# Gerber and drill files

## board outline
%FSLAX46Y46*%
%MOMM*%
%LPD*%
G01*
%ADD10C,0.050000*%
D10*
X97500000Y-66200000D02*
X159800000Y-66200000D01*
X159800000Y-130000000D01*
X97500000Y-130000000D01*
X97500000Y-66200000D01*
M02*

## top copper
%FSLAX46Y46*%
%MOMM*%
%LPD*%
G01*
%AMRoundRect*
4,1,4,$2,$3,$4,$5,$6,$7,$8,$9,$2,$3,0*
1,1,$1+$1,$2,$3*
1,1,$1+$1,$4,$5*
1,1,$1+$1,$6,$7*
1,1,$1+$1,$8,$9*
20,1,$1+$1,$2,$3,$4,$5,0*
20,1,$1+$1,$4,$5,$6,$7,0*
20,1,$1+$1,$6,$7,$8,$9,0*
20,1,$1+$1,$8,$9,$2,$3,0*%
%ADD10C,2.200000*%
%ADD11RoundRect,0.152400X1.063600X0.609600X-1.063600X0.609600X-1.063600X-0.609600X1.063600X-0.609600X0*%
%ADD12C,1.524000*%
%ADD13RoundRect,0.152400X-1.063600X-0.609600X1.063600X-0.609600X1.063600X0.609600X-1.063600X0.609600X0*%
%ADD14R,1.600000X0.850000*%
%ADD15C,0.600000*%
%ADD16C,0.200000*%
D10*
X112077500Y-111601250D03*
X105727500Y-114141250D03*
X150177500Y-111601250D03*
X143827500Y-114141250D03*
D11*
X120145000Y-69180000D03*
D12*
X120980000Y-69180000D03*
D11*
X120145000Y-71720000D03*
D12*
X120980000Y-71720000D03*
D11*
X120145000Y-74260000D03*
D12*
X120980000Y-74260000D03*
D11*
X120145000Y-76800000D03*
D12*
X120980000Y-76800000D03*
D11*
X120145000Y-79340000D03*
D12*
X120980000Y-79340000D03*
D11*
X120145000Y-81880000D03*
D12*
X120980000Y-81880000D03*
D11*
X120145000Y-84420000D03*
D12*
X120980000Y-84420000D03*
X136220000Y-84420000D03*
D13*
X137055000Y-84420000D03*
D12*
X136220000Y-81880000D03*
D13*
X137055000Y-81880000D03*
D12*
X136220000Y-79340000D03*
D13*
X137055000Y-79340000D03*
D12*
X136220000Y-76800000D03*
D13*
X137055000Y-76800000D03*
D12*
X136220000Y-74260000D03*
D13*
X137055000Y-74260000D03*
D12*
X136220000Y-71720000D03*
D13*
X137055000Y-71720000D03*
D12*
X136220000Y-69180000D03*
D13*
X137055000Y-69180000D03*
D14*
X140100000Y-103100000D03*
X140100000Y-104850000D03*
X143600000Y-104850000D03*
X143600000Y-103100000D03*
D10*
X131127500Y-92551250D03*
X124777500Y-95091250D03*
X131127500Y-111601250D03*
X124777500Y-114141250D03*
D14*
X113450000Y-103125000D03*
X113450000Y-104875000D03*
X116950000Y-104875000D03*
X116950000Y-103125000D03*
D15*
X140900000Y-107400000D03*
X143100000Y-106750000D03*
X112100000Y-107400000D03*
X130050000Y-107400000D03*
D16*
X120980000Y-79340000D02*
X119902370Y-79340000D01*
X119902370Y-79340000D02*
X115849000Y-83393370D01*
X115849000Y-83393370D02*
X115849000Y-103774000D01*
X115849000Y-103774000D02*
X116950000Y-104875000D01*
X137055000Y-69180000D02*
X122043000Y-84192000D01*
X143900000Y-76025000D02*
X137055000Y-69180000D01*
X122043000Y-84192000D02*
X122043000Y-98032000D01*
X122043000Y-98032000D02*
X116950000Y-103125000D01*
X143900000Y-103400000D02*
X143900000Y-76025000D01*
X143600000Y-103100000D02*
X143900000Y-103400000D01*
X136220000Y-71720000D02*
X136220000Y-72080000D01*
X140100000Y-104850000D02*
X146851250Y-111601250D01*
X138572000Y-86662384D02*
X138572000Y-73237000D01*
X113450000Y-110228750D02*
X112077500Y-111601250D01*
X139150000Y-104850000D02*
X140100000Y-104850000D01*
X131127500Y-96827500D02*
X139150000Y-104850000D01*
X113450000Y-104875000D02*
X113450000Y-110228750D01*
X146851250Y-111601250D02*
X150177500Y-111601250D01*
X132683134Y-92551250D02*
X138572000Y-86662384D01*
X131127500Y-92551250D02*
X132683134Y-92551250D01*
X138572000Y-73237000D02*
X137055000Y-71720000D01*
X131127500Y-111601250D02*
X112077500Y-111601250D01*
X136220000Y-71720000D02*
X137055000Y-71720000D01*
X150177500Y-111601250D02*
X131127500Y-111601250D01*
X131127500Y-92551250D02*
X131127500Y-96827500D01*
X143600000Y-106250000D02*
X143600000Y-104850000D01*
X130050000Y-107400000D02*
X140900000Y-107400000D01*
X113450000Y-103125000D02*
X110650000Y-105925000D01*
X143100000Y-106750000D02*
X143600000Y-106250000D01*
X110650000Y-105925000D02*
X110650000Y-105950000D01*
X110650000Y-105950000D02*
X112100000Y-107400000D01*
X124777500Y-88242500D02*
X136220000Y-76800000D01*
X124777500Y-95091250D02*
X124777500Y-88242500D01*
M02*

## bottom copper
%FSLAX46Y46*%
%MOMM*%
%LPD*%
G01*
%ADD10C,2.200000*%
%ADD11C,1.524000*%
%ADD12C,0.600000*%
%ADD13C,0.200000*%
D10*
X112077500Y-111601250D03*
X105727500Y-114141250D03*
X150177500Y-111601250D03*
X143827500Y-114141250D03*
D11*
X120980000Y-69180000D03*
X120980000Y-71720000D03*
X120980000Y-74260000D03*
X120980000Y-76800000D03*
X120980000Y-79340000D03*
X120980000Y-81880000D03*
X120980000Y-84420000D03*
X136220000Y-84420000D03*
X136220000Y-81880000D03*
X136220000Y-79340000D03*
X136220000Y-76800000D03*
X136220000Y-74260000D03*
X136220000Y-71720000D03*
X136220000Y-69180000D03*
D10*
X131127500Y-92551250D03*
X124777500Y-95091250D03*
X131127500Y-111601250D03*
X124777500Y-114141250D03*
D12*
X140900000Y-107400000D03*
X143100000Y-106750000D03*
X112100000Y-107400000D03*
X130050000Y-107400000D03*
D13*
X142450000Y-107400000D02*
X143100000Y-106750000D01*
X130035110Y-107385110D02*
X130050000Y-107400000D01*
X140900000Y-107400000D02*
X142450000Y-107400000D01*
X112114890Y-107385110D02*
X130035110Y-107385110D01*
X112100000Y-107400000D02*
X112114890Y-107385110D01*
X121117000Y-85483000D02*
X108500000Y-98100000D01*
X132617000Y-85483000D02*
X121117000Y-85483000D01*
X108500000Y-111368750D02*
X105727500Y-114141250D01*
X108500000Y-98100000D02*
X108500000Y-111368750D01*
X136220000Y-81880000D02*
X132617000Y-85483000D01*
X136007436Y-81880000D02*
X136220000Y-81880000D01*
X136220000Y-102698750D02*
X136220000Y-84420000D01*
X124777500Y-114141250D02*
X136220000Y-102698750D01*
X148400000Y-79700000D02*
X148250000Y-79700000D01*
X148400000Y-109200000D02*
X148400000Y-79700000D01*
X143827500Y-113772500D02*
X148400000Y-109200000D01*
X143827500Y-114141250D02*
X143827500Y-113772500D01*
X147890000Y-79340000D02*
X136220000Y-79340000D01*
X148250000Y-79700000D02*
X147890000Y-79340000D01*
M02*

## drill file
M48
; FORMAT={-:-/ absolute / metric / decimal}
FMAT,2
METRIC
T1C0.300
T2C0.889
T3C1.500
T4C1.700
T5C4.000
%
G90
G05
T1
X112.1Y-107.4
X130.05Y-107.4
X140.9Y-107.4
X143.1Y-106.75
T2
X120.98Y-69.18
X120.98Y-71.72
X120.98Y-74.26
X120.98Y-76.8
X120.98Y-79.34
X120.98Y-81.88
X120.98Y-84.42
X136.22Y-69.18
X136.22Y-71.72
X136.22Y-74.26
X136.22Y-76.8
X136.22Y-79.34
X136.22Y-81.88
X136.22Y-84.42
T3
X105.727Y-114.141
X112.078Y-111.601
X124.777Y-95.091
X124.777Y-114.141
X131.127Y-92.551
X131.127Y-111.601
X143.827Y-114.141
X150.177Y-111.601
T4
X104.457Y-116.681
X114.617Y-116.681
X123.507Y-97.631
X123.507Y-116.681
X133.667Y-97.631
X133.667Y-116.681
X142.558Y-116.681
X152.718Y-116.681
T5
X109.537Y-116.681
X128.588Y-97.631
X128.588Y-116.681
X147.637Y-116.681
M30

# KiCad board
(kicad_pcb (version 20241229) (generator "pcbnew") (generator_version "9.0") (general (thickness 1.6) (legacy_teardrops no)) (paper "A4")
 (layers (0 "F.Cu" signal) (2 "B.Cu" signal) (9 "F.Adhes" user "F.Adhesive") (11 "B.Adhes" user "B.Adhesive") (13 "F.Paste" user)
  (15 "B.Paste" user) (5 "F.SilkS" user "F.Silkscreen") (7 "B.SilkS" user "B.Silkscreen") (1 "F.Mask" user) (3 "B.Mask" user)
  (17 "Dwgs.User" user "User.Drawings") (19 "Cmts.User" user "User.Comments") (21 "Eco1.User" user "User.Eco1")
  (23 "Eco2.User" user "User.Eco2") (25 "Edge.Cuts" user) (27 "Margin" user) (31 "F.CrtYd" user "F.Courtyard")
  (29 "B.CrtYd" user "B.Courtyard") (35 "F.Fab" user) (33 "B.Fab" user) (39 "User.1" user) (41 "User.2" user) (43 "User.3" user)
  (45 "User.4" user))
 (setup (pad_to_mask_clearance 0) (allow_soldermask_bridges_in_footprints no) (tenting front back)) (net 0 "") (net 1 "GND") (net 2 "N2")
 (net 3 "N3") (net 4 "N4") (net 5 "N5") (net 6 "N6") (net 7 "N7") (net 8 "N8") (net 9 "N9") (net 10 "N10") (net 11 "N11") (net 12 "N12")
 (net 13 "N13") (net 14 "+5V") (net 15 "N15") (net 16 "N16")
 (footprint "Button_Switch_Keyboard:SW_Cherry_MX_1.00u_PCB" (layer "F.Cu") (at 112.0775 111.60125)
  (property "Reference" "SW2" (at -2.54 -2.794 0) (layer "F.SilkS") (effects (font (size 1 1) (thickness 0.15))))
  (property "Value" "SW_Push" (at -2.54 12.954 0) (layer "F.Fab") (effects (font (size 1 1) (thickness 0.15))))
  (pad "" np_thru_hole circle (at -7.62 5.08) (size 1.7 1.7) (drill 1.7) (layers "*.Cu" "*.Mask"))
  (pad "" np_thru_hole circle (at -2.54 5.08) (size 4 4) (drill 4) (layers "*.Cu" "*.Mask"))
  (pad "" np_thru_hole circle (at 2.54 5.08) (size 1.7 1.7) (drill 1.7) (layers "*.Cu" "*.Mask"))
  (pad "1" thru_hole circle (at 0 0) (size 2.2 2.2) (drill 1.5) (layers "*.Cu" "*.Mask") (remove_unused_layers no) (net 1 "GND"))
  (pad "2" thru_hole circle (at -6.35 2.54) (size 2.2 2.2) (drill 1.5) (layers "*.Cu" "*.Mask") (remove_unused_layers no) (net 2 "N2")))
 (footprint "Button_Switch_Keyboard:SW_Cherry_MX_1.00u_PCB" (layer "F.Cu") (at 150.1775 111.60125)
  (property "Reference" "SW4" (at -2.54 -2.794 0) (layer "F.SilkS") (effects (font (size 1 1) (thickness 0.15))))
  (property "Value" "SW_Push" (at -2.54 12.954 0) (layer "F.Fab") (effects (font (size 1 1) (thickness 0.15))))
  (pad "" np_thru_hole circle (at -7.62 5.08) (size 1.7 1.7) (drill 1.7) (layers "*.Cu" "*.Mask"))
  (pad "" np_thru_hole circle (at -2.54 5.08) (size 4 4) (drill 4) (layers "*.Cu" "*.Mask"))
  (pad "" np_thru_hole circle (at 2.54 5.08) (size 1.7 1.7) (drill 1.7) (layers "*.Cu" "*.Mask"))
  (pad "1" thru_hole circle (at 0 0) (size 2.2 2.2) (drill 1.5) (layers "*.Cu" "*.Mask") (remove_unused_layers no) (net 1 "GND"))
  (pad "2" thru_hole circle (at -6.35 2.54) (size 2.2 2.2) (drill 1.5) (layers "*.Cu" "*.Mask") (remove_unused_layers no) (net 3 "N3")))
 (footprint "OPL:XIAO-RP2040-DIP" (layer "F.Cu") (at 128.6 76.8)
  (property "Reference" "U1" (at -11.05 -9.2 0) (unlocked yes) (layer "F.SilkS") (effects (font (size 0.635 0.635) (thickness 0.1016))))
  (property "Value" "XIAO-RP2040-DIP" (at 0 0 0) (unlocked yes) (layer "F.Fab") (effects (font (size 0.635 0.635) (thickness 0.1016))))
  (pad "1" smd roundrect (at -8.455 -7.62 180) (size 2.432 1.524) (layers "F.Cu" "F.Mask") (roundrect_rratio 0.1) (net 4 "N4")
   (thermal_bridge_angle 45))
  (pad "1" thru_hole circle (at -7.62 -7.62 180) (size 1.524 1.524) (drill 0.889) (layers "*.Cu" "*.Mask") (remove_unused_layers no)
   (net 4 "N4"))
  (pad "2" smd roundrect (at -8.455 -5.08 180) (size 2.432 1.524) (layers "F.Cu" "F.Mask") (roundrect_rratio 0.1) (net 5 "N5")
   (thermal_bridge_angle 45))
  (pad "2" thru_hole circle (at -7.62 -5.08 180) (size 1.524 1.524) (drill 0.889) (layers "*.Cu" "*.Mask") (remove_unused_layers no)
   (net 5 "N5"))
  (pad "3" smd roundrect (at -8.455 -2.54 180) (size 2.432 1.524) (layers "F.Cu" "F.Mask") (roundrect_rratio 0.1) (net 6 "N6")
   (thermal_bridge_angle 45))
  (pad "3" thru_hole circle (at -7.62 -2.54 180) (size 1.524 1.524) (drill 0.889) (layers "*.Cu" "*.Mask") (remove_unused_layers no)
   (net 6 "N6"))
  (pad "4" smd roundrect (at -8.455 0 180) (size 2.432 1.524) (layers "F.Cu" "F.Mask") (roundrect_rratio 0.1) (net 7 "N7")
   (thermal_bridge_angle 45))
  (pad "4" thru_hole circle (at -7.62 0 180) (size 1.524 1.524) (drill 0.889) (layers "*.Cu" "*.Mask") (remove_unused_layers no)
   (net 7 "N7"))
  (pad "5" smd roundrect (at -8.455 2.54 180) (size 2.432 1.524) (layers "F.Cu" "F.Mask") (roundrect_rratio 0.1) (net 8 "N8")
   (thermal_bridge_angle 45))
  (pad "5" thru_hole circle (at -7.62 2.54 180) (size 1.524 1.524) (drill 0.889) (layers "*.Cu" "*.Mask") (remove_unused_layers no)
   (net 8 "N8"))
  (pad "6" smd roundrect (at -8.455 5.08 180) (size 2.432 1.524) (layers "F.Cu" "F.Mask") (roundrect_rratio 0.1) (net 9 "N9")
   (thermal_bridge_angle 45))
  (pad "6" thru_hole circle (at -7.62 5.08 180) (size 1.524 1.524) (drill 0.889) (layers "*.Cu" "*.Mask") (remove_unused_layers no)
   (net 9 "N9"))
  (pad "7" smd roundrect (at -8.455 7.62 180) (size 2.432 1.524) (layers "F.Cu" "F.Mask") (roundrect_rratio 0.1) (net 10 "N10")
   (thermal_bridge_angle 45))
  (pad "7" thru_hole circle (at -7.62 7.62 180) (size 1.524 1.524) (drill 0.889) (layers "*.Cu" "*.Mask") (remove_unused_layers no)
   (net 10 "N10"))
  (pad "8" thru_hole circle (at 7.62 7.62) (size 1.524 1.524) (drill 0.889) (layers "*.Cu" "*.Mask") (remove_unused_layers no)
   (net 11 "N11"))
  (pad "8" smd roundrect (at 8.455 7.62) (size 2.432 1.524) (layers "F.Cu" "F.Mask") (roundrect_rratio 0.1) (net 11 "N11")
   (thermal_bridge_angle 45))
  (pad "9" thru_hole circle (at 7.62 5.08) (size 1.524 1.524) (drill 0.889) (layers "*.Cu" "*.Mask") (remove_unused_layers no) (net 2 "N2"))
  (pad "9" smd roundrect (at 8.455 5.08) (size 2.432 1.524) (layers "F.Cu" "F.Mask") (roundrect_rratio 0.1) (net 2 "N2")
   (thermal_bridge_angle 45))
  (pad "10" thru_hole circle (at 7.62 2.54) (size 1.524 1.524) (drill 0.889) (layers "*.Cu" "*.Mask") (remove_unused_layers no) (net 3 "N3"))
  (pad "10" smd roundrect (at 8.455 2.54) (size 2.432 1.524) (layers "F.Cu" "F.Mask") (roundrect_rratio 0.1) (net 3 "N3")
   (thermal_bridge_angle 45))
  (pad "11" thru_hole circle (at 7.62 0) (size 1.524 1.524) (drill 0.889) (layers "*.Cu" "*.Mask") (remove_unused_layers no) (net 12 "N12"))
  (pad "11" smd roundrect (at 8.455 0) (size 2.432 1.524) (layers "F.Cu" "F.Mask") (roundrect_rratio 0.1) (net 12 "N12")
   (thermal_bridge_angle 45))
  (pad "12" thru_hole circle (at 7.62 -2.54) (size 1.524 1.524) (drill 0.889) (layers "*.Cu" "*.Mask") (remove_unused_layers no)
   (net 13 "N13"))
  (pad "12" smd roundrect (at 8.455 -2.54) (size 2.432 1.524) (layers "F.Cu" "F.Mask") (roundrect_rratio 0.1) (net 13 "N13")
   (thermal_bridge_angle 45))
  (pad "13" thru_hole circle (at 7.62 -5.08) (size 1.524 1.524) (drill 0.889) (layers "*.Cu" "*.Mask") (remove_unused_layers no)
   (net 1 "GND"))
  (pad "13" smd roundrect (at 8.455 -5.08) (size 2.432 1.524) (layers "F.Cu" "F.Mask") (roundrect_rratio 0.1) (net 1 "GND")
   (thermal_bridge_angle 45))
  (pad "14" thru_hole circle (at 7.62 -7.62) (size 1.524 1.524) (drill 0.889) (layers "*.Cu" "*.Mask") (remove_unused_layers no)
   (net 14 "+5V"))
  (pad "14" smd roundrect (at 8.455 -7.62) (size 2.432 1.524) (layers "F.Cu" "F.Mask") (roundrect_rratio 0.1) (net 14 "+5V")
   (thermal_bridge_angle 45)))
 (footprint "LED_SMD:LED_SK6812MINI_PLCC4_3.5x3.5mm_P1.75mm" (layer "F.Cu") (at 141.85 103.975)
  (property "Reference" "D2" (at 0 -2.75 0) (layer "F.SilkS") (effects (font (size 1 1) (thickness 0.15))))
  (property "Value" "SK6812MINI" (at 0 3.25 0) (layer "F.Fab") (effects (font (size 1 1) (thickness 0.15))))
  (pad "1" smd rect (at -1.75 -0.875) (size 1.6 0.85) (layers "F.Cu" "F.Mask" "F.Paste") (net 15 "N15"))
  (pad "2" smd rect (at -1.75 0.875) (size 1.6 0.85) (layers "F.Cu" "F.Mask" "F.Paste") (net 1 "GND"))
  (pad "3" smd rect (at 1.75 0.875) (size 1.6 0.85) (layers "F.Cu" "F.Mask" "F.Paste") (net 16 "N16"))
  (pad "4" smd rect (at 1.75 -0.875) (size 1.6 0.85) (layers "F.Cu" "F.Mask" "F.Paste") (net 14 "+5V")))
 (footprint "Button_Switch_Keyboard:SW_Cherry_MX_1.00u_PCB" (layer "F.Cu") (at 131.1275 92.55125)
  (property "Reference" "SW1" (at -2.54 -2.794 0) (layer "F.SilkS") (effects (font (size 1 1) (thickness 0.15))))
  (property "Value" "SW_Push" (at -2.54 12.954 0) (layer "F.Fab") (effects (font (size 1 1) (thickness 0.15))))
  (pad "" np_thru_hole circle (at -7.62 5.08) (size 1.7 1.7) (drill 1.7) (layers "*.Cu" "*.Mask"))
  (pad "" np_thru_hole circle (at -2.54 5.08) (size 4 4) (drill 4) (layers "*.Cu" "*.Mask"))
  (pad "" np_thru_hole circle (at 2.54 5.08) (size 1.7 1.7) (drill 1.7) (layers "*.Cu" "*.Mask"))
  (pad "1" thru_hole circle (at 0 0) (size 2.2 2.2) (drill 1.5) (layers "*.Cu" "*.Mask") (remove_unused_layers no) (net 1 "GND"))
  (pad "2" thru_hole circle (at -6.35 2.54) (size 2.2 2.2) (drill 1.5) (layers "*.Cu" "*.Mask") (remove_unused_layers no) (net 12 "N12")))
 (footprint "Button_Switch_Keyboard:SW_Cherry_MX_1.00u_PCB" (layer "F.Cu") (at 131.1275 111.60125)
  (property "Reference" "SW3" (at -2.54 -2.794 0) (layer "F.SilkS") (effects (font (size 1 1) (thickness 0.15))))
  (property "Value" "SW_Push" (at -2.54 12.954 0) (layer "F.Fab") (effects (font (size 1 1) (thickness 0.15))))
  (pad "" np_thru_hole circle (at -7.62 5.08) (size 1.7 1.7) (drill 1.7) (layers "*.Cu" "*.Mask"))
  (pad "" np_thru_hole circle (at -2.54 5.08) (size 4 4) (drill 4) (layers "*.Cu" "*.Mask"))
  (pad "" np_thru_hole circle (at 2.54 5.08) (size 1.7 1.7) (drill 1.7) (layers "*.Cu" "*.Mask"))
  (pad "1" thru_hole circle (at 0 0) (size 2.2 2.2) (drill 1.5) (layers "*.Cu" "*.Mask") (remove_unused_layers no) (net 1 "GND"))
  (pad "2" thru_hole circle (at -6.35 2.54) (size 2.2 2.2) (drill 1.5) (layers "*.Cu" "*.Mask") (remove_unused_layers no) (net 11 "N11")))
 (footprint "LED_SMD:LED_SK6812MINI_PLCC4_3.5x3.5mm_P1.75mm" (layer "F.Cu") (at 115.2 104)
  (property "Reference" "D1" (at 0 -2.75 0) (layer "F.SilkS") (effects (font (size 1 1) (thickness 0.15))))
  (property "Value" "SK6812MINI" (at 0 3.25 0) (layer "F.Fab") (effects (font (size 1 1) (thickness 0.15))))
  (pad "1" smd rect (at -1.75 -0.875) (size 1.6 0.85) (layers "F.Cu" "F.Mask" "F.Paste") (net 16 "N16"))
  (pad "2" smd rect (at -1.75 0.875) (size 1.6 0.85) (layers "F.Cu" "F.Mask" "F.Paste") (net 1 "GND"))
  (pad "3" smd rect (at 1.75 0.875) (size 1.6 0.85) (layers "F.Cu" "F.Mask" "F.Paste") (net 8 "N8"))
  (pad "4" smd rect (at 1.75 -0.875) (size 1.6 0.85) (layers "F.Cu" "F.Mask" "F.Paste") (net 14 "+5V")))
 (gr_rect (start 97.5 66.2) (end 159.8 130) (stroke (width 0.05) (type default)) (fill no) (layer "Edge.Cuts"))
 (segment (start 120.98 79.34) (end 119.90237 79.34) (width 0.2) (layer "F.Cu") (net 8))
 (segment (start 119.90237 79.34) (end 115.849 83.39337) (width 0.2) (layer "F.Cu") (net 8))
 (segment (start 115.849 83.39337) (end 115.849 103.774) (width 0.2) (layer "F.Cu") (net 8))
 (segment (start 115.849 103.774) (end 116.95 104.875) (width 0.2) (layer "F.Cu") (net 8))
 (segment (start 137.055 69.18) (end 122.043 84.192) (width 0.2) (layer "F.Cu") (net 14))
 (segment (start 143.9 76.025) (end 137.055 69.18) (width 0.2) (layer "F.Cu") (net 14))
 (segment (start 122.043 84.192) (end 122.043 98.032) (width 0.2) (layer "F.Cu") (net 14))
 (segment (start 122.043 98.032) (end 116.95 103.125) (width 0.2) (layer "F.Cu") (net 14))
 (segment (start 143.9 103.4) (end 143.9 76.025) (width 0.2) (layer "F.Cu") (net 14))
 (segment (start 143.6 103.1) (end 143.9 103.4) (width 0.2) (layer "F.Cu") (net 14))
 (segment (start 136.22 71.72) (end 136.22 72.08) (width 0.2) (layer "F.Cu") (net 1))
 (segment (start 140.1 104.85) (end 146.85125 111.60125) (width 0.2) (layer "F.Cu") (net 1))
 (segment (start 138.572 86.662384) (end 138.572 73.237) (width 0.2) (layer "F.Cu") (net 1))
 (segment (start 113.45 110.22875) (end 112.0775 111.60125) (width 0.2) (layer "F.Cu") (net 1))
 (segment (start 139.15 104.85) (end 140.1 104.85) (width 0.2) (layer "F.Cu") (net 1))
 (segment (start 131.1275 96.8275) (end 139.15 104.85) (width 0.2) (layer "F.Cu") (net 1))
 (segment (start 113.45 104.875) (end 113.45 110.22875) (width 0.2) (layer "F.Cu") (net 1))
 (segment (start 146.85125 111.60125) (end 150.1775 111.60125) (width 0.2) (layer "F.Cu") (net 1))
 (segment (start 132.683134 92.55125) (end 138.572 86.662384) (width 0.2) (layer "F.Cu") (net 1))
 (segment (start 131.1275 92.55125) (end 132.683134 92.55125) (width 0.2) (layer "F.Cu") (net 1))
 (segment (start 138.572 73.237) (end 137.055 71.72) (width 0.2) (layer "F.Cu") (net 1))
 (segment (start 131.1275 111.60125) (end 112.0775 111.60125) (width 0.2) (layer "F.Cu") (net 1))
 (segment (start 136.22 71.72) (end 137.055 71.72) (width 0.2) (layer "F.Cu") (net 1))
 (segment (start 150.1775 111.60125) (end 131.1275 111.60125) (width 0.2) (layer "F.Cu") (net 1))
 (segment (start 131.1275 92.55125) (end 131.1275 96.8275) (width 0.2) (layer "F.Cu") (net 1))
 (segment (start 143.6 106.25) (end 143.6 104.85) (width 0.2) (layer "F.Cu") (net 16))
 (segment (start 130.05 107.4) (end 140.9 107.4) (width 0.2) (layer "F.Cu") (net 16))
 (segment (start 113.45 103.125) (end 110.65 105.925) (width 0.2) (layer "F.Cu") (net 16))
 (segment (start 143.1 106.75) (end 143.6 106.25) (width 0.2) (layer "F.Cu") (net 16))
 (segment (start 110.65 105.925) (end 110.65 105.95) (width 0.2) (layer "F.Cu") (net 16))
 (segment (start 110.65 105.95) (end 112.1 107.4) (width 0.2) (layer "F.Cu") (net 16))
 (via (at 140.9 107.4) (size 0.6) (drill 0.3) (layers "F.Cu" "B.Cu") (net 16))
 (via (at 143.1 106.75) (size 0.6) (drill 0.3) (layers "F.Cu" "B.Cu") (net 16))
 (via (at 112.1 107.4) (size 0.6) (drill 0.3) (layers "F.Cu" "B.Cu") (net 16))
 (via (at 130.05 107.4) (size 0.6) (drill 0.3) (layers "F.Cu" "B.Cu") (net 16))
 (segment (start 142.45 107.4) (end 143.1 106.75) (width 0.2) (layer "B.Cu") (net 16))
 (segment (start 130.03511 107.38511) (end 130.05 107.4) (width 0.2) (layer "B.Cu") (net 16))
 (segment (start 140.9 107.4) (end 142.45 107.4) (width 0.2) (layer "B.Cu") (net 16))
 (segment (start 112.11489 107.38511) (end 130.03511 107.38511) (width 0.2) (layer "B.Cu") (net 16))
 (segment (start 112.1 107.4) (end 112.11489 107.38511) (width 0.2) (layer "B.Cu") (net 16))
 (segment (start 124.7775 88.2425) (end 136.22 76.8) (width 0.2) (layer "F.Cu") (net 12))
 (segment (start 124.7775 95.09125) (end 124.7775 88.2425) (width 0.2) (layer "F.Cu") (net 12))
 (segment (start 121.117 85.483) (end 108.5 98.1) (width 0.2) (layer "B.Cu") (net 2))
 (segment (start 132.617 85.483) (end 121.117 85.483) (width 0.2) (layer "B.Cu") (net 2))
 (segment (start 108.5 111.36875) (end 105.7275 114.14125) (width 0.2) (layer "B.Cu") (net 2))
 (segment (start 108.5 98.1) (end 108.5 111.36875) (width 0.2) (layer "B.Cu") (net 2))
 (segment (start 136.22 81.88) (end 132.617 85.483) (width 0.2) (layer "B.Cu") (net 2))
 (segment (start 136.007436 81.88) (end 136.22 81.88) (width 0.2) (layer "B.Cu") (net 2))
 (segment (start 136.22 102.69875) (end 136.22 84.42) (width 0.2) (layer "B.Cu") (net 11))
 (segment (start 124.7775 114.14125) (end 136.22 102.69875) (width 0.2) (layer "B.Cu") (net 11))
 (segment (start 148.4 79.7) (end 148.25 79.7) (width 0.2) (layer "B.Cu") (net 3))
 (segment (start 148.4 109.2) (end 148.4 79.7) (width 0.2) (layer "B.Cu") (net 3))
 (segment (start 143.8275 113.7725) (end 148.4 109.2) (width 0.2) (layer "B.Cu") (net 3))
 (segment (start 143.8275 114.14125) (end 143.8275 113.7725) (width 0.2) (layer "B.Cu") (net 3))
 (segment (start 147.89 79.34) (end 136.22 79.34) (width 0.2) (layer "B.Cu") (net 3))
 (segment (start 148.25 79.7) (end 147.89 79.34) (width 0.2) (layer "B.Cu") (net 3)))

